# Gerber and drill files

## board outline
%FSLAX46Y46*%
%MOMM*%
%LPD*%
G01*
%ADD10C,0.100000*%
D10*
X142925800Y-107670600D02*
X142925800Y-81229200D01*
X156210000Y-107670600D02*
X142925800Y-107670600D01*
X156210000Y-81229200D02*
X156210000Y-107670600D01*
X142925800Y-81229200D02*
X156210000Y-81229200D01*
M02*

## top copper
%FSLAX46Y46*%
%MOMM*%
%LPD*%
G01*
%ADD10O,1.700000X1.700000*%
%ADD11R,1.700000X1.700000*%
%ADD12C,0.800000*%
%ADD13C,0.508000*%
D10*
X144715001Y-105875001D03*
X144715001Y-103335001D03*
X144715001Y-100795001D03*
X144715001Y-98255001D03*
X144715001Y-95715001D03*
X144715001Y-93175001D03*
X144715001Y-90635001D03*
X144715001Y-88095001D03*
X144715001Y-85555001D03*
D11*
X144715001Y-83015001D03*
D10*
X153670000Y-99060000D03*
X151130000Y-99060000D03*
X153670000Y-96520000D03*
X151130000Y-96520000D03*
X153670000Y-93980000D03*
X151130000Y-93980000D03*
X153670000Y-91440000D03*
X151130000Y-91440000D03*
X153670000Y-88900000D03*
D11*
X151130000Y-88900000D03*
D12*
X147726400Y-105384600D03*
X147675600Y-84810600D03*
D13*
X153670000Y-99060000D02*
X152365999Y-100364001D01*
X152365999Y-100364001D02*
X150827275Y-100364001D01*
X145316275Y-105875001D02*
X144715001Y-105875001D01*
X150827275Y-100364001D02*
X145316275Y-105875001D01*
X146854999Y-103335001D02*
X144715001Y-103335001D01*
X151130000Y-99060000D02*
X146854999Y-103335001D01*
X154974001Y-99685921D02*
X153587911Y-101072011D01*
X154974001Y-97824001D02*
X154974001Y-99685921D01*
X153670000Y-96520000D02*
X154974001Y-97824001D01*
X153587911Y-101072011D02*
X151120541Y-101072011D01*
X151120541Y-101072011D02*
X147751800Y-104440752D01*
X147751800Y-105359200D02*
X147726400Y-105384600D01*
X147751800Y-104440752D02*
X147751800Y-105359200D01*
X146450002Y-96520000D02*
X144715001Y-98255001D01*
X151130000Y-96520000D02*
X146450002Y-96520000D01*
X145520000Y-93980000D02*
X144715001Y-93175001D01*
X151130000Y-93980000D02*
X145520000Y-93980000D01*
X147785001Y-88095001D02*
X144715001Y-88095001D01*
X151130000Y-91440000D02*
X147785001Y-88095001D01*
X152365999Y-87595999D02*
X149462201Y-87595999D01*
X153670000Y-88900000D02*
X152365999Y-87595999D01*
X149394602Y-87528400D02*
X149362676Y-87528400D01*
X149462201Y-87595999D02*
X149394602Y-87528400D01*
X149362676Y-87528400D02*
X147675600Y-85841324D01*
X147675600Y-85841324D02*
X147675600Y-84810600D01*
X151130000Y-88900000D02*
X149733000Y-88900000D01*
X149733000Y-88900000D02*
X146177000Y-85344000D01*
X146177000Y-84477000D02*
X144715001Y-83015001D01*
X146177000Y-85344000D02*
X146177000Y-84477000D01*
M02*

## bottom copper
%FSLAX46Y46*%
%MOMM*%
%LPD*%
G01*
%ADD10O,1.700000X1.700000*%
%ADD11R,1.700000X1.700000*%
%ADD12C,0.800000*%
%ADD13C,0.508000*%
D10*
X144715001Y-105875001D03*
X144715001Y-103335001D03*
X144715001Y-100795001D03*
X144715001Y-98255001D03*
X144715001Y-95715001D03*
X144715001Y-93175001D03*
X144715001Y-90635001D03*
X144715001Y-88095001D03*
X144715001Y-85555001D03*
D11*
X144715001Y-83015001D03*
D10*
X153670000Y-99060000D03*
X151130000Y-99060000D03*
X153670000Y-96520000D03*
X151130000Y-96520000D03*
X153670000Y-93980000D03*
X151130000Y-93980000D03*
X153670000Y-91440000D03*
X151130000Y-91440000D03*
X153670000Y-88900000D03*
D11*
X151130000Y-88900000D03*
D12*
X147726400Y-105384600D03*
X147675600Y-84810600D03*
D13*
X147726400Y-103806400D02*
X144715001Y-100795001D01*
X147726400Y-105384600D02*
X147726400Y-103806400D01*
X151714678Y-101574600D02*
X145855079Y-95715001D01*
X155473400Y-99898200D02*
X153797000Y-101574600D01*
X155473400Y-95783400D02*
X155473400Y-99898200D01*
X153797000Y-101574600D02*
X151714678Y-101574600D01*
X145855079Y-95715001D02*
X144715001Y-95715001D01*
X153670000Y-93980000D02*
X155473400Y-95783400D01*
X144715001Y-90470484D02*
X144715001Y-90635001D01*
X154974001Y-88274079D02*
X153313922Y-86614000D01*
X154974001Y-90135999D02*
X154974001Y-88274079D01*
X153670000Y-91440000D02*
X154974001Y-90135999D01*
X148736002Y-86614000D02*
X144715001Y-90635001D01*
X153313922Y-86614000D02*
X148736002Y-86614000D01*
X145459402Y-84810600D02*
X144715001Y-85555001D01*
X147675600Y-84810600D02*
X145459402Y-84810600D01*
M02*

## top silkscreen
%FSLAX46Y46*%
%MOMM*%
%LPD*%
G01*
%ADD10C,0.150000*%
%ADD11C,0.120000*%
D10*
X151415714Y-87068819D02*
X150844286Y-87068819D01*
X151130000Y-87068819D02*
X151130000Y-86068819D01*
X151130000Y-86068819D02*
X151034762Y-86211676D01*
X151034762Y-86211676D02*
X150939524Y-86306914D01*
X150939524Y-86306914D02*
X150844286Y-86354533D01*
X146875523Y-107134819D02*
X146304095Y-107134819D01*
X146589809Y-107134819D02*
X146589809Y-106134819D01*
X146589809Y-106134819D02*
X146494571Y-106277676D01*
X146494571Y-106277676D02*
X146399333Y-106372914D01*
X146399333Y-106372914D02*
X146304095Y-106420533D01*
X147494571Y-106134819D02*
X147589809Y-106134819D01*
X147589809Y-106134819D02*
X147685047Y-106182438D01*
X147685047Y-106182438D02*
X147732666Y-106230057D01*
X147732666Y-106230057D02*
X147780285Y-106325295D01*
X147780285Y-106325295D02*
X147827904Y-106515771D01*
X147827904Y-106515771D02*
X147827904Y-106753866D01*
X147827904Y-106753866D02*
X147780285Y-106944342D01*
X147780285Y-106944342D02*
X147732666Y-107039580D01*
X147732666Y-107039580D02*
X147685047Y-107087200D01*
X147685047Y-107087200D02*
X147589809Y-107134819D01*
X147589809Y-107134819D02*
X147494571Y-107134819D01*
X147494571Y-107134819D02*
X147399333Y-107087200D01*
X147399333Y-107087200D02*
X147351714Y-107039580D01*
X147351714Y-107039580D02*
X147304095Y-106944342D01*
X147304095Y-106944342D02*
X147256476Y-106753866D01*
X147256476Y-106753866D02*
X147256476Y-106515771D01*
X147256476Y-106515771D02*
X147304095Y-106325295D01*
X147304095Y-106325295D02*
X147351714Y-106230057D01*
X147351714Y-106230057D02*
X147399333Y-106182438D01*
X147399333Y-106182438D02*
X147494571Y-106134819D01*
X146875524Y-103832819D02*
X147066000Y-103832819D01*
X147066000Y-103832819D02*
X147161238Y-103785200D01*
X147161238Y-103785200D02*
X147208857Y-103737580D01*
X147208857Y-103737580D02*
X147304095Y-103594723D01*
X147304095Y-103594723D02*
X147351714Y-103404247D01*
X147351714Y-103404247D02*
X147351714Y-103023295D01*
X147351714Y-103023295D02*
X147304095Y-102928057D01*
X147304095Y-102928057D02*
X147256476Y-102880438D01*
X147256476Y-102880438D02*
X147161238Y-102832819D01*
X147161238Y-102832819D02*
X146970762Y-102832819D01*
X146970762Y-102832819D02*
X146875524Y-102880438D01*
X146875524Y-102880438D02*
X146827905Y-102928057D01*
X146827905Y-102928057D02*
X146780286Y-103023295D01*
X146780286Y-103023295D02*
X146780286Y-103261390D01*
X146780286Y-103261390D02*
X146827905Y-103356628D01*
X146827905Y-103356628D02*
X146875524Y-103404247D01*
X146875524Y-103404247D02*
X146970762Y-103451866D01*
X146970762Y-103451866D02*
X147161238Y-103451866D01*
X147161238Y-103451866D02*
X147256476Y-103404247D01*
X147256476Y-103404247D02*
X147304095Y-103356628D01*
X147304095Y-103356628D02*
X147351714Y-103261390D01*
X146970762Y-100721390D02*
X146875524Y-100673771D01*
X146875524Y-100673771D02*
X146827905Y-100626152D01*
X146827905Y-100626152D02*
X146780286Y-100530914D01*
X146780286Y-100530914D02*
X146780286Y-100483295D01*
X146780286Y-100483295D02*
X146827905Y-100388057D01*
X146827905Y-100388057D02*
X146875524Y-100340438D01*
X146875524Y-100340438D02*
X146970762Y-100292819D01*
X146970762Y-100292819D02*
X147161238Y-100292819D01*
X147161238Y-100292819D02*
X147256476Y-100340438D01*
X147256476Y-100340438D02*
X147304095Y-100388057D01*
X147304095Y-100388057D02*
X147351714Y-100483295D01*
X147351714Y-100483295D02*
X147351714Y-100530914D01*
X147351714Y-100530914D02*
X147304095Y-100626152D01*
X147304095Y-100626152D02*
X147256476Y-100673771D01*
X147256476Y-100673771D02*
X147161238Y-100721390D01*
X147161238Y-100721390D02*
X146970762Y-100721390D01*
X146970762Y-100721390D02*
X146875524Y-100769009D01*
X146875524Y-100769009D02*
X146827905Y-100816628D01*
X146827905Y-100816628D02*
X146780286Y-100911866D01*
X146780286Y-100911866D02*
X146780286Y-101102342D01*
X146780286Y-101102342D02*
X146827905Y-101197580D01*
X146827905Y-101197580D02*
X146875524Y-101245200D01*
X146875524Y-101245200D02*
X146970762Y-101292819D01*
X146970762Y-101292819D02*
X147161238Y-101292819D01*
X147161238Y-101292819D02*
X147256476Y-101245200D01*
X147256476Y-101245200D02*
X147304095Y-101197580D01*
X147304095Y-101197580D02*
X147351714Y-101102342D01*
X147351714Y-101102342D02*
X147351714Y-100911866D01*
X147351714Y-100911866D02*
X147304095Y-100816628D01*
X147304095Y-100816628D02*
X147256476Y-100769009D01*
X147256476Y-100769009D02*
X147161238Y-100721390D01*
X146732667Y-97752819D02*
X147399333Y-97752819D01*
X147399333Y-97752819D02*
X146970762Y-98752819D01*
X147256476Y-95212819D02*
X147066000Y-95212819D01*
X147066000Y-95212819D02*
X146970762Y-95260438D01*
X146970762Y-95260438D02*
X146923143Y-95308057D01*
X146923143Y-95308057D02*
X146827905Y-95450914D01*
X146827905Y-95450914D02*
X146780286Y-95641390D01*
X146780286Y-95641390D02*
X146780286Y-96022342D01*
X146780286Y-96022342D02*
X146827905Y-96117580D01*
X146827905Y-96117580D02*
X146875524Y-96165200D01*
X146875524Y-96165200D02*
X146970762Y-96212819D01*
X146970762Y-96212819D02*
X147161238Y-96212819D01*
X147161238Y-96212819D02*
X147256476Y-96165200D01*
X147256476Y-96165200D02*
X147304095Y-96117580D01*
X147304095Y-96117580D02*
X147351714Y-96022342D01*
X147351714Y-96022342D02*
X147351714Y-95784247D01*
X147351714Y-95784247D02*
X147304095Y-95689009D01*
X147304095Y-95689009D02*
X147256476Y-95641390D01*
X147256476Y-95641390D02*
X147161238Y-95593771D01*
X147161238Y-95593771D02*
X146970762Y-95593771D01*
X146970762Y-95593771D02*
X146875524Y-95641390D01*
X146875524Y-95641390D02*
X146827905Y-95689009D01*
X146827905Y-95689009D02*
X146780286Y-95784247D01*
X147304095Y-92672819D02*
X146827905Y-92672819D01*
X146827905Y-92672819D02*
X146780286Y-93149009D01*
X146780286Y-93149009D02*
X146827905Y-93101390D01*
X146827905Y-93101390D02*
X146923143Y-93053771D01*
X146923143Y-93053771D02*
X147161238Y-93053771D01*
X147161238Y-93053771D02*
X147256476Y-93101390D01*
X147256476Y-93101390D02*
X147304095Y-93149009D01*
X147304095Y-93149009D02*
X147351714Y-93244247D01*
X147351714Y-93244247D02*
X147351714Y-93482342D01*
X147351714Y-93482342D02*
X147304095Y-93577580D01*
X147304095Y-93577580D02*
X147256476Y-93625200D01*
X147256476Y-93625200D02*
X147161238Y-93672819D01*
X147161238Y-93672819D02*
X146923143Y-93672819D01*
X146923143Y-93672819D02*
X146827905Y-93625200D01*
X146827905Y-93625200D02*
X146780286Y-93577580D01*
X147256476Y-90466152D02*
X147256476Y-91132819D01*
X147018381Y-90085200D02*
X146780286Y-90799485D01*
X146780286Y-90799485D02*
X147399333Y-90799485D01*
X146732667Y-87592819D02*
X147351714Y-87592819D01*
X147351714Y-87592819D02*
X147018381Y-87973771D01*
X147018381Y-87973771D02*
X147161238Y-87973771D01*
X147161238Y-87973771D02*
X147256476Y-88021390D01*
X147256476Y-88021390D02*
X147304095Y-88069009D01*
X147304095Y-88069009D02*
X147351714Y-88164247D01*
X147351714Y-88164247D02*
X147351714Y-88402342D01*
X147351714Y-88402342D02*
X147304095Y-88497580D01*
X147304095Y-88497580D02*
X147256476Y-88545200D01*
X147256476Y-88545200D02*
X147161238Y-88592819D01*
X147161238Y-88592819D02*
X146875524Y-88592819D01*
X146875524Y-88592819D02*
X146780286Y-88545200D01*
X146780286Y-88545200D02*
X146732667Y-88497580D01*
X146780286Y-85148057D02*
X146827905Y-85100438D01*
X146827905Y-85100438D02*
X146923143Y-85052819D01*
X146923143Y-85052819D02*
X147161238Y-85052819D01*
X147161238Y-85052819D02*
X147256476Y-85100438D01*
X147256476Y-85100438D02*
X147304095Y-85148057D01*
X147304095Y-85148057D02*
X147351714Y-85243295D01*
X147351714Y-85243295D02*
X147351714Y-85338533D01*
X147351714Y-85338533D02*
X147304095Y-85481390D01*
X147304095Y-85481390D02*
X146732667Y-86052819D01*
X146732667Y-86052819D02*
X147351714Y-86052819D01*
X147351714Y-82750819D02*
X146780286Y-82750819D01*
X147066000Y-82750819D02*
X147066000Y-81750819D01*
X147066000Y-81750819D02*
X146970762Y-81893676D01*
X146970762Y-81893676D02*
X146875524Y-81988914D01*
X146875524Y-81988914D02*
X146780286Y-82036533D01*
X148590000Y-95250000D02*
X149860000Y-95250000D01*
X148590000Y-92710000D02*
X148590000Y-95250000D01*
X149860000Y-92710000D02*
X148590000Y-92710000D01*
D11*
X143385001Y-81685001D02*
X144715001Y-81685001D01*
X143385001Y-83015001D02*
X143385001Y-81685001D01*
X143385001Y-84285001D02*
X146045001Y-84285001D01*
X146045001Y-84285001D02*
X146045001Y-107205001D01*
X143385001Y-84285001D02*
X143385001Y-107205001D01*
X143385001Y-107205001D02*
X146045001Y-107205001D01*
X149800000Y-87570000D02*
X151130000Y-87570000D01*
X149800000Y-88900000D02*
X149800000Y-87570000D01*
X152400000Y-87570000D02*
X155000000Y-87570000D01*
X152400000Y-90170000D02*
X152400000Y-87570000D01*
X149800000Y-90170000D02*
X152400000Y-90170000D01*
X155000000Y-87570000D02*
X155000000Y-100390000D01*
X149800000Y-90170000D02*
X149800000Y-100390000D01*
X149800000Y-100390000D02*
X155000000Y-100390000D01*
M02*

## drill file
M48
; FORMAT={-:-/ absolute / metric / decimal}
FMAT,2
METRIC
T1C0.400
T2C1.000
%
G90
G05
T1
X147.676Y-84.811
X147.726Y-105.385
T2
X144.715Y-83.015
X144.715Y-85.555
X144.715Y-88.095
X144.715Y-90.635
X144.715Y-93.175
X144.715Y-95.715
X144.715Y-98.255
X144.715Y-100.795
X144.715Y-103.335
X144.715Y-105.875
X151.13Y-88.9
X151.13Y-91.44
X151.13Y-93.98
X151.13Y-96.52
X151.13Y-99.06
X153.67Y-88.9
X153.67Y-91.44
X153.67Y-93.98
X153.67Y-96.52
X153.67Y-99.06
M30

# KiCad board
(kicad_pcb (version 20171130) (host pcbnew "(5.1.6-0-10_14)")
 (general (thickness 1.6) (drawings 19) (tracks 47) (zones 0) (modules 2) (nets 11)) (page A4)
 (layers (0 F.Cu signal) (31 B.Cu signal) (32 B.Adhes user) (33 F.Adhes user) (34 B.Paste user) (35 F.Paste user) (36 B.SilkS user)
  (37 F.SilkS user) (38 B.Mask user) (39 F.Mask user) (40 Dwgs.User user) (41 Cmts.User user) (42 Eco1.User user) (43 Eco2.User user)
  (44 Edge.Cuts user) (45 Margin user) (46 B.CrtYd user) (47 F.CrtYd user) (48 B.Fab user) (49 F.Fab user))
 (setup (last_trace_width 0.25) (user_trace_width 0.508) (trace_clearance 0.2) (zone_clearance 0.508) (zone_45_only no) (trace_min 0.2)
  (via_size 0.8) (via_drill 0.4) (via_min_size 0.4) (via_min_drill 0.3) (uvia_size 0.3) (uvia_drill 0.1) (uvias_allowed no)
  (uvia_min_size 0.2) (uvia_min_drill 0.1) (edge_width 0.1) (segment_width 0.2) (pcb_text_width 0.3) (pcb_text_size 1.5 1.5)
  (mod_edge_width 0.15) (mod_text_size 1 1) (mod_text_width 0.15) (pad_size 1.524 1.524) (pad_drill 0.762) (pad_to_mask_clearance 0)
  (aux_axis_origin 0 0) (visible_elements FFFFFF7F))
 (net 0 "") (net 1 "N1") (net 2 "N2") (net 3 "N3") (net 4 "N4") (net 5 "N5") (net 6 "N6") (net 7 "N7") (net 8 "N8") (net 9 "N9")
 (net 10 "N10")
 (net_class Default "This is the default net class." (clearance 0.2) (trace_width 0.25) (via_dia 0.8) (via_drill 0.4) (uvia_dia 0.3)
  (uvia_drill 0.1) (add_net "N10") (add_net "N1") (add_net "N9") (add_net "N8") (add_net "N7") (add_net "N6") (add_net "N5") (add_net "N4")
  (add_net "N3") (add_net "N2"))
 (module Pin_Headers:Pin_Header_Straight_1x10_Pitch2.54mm (layer F.Cu) (at 144.715001 83.015001)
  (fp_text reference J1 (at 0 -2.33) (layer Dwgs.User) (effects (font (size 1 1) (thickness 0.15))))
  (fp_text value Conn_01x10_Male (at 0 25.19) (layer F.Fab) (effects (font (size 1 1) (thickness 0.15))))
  (fp_line (start -1.33 -1.33) (end 0 -1.33) (layer F.SilkS) (width 0.12))
  (fp_line (start -1.33 0) (end -1.33 -1.33) (layer F.SilkS) (width 0.12))
  (fp_line (start -1.33 1.27) (end 1.33 1.27) (layer F.SilkS) (width 0.12))
  (fp_line (start 1.33 1.27) (end 1.33 24.19) (layer F.SilkS) (width 0.12))
  (fp_line (start -1.33 1.27) (end -1.33 24.19) (layer F.SilkS) (width 0.12))
  (fp_line (start -1.33 24.19) (end 1.33 24.19) (layer F.SilkS) (width 0.12))
  (pad 10 thru_hole oval (at 0 22.86) (size 1.7 1.7) (drill 1) (layers *.Cu *.Mask) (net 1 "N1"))
  (pad 9 thru_hole oval (at 0 20.32) (size 1.7 1.7) (drill 1) (layers *.Cu *.Mask) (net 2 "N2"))
  (pad 8 thru_hole oval (at 0 17.78) (size 1.7 1.7) (drill 1) (layers *.Cu *.Mask) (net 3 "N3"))
  (pad 7 thru_hole oval (at 0 15.24) (size 1.7 1.7) (drill 1) (layers *.Cu *.Mask) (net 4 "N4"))
  (pad 6 thru_hole oval (at 0 12.7) (size 1.7 1.7) (drill 1) (layers *.Cu *.Mask) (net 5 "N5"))
  (pad 5 thru_hole oval (at 0 10.16) (size 1.7 1.7) (drill 1) (layers *.Cu *.Mask) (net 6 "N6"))
  (pad 4 thru_hole oval (at 0 7.62) (size 1.7 1.7) (drill 1) (layers *.Cu *.Mask) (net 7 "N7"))
  (pad 3 thru_hole oval (at 0 5.08) (size 1.7 1.7) (drill 1) (layers *.Cu *.Mask) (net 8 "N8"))
  (pad 2 thru_hole oval (at 0 2.54) (size 1.7 1.7) (drill 1) (layers *.Cu *.Mask) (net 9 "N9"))
  (pad 1 thru_hole rect (at 0 0) (size 1.7 1.7) (drill 1) (layers *.Cu *.Mask) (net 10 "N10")))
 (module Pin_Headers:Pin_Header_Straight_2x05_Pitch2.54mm (layer F.Cu) (at 151.13 88.9)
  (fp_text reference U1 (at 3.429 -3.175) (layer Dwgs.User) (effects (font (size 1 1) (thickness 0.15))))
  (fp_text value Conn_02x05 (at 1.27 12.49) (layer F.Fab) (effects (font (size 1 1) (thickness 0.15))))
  (fp_line (start -1.33 -1.33) (end 0 -1.33) (layer F.SilkS) (width 0.12))
  (fp_line (start -1.33 0) (end -1.33 -1.33) (layer F.SilkS) (width 0.12))
  (fp_line (start 1.27 -1.33) (end 3.87 -1.33) (layer F.SilkS) (width 0.12))
  (fp_line (start 1.27 1.27) (end 1.27 -1.33) (layer F.SilkS) (width 0.12))
  (fp_line (start -1.33 1.27) (end 1.27 1.27) (layer F.SilkS) (width 0.12))
  (fp_line (start 3.87 -1.33) (end 3.87 11.49) (layer F.SilkS) (width 0.12))
  (fp_line (start -1.33 1.27) (end -1.33 11.49) (layer F.SilkS) (width 0.12))
  (fp_line (start -1.33 11.49) (end 3.87 11.49) (layer F.SilkS) (width 0.12))
  (pad 10 thru_hole oval (at 2.54 10.16) (size 1.7 1.7) (drill 1) (layers *.Cu *.Mask) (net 1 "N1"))
  (pad 9 thru_hole oval (at 0 10.16) (size 1.7 1.7) (drill 1) (layers *.Cu *.Mask) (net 2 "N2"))
  (pad 8 thru_hole oval (at 2.54 7.62) (size 1.7 1.7) (drill 1) (layers *.Cu *.Mask) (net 3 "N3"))
  (pad 7 thru_hole oval (at 0 7.62) (size 1.7 1.7) (drill 1) (layers *.Cu *.Mask) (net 4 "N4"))
  (pad 6 thru_hole oval (at 2.54 5.08) (size 1.7 1.7) (drill 1) (layers *.Cu *.Mask) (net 5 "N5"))
  (pad 5 thru_hole oval (at 0 5.08) (size 1.7 1.7) (drill 1) (layers *.Cu *.Mask) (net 6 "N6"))
  (pad 4 thru_hole oval (at 2.54 2.54) (size 1.7 1.7) (drill 1) (layers *.Cu *.Mask) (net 7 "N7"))
  (pad 3 thru_hole oval (at 0 2.54) (size 1.7 1.7) (drill 1) (layers *.Cu *.Mask) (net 8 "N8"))
  (pad 2 thru_hole oval (at 2.54 0) (size 1.7 1.7) (drill 1) (layers *.Cu *.Mask) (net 9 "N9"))
  (pad 1 thru_hole rect (at 0 0) (size 1.7 1.7) (drill 1) (layers *.Cu *.Mask) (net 10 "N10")))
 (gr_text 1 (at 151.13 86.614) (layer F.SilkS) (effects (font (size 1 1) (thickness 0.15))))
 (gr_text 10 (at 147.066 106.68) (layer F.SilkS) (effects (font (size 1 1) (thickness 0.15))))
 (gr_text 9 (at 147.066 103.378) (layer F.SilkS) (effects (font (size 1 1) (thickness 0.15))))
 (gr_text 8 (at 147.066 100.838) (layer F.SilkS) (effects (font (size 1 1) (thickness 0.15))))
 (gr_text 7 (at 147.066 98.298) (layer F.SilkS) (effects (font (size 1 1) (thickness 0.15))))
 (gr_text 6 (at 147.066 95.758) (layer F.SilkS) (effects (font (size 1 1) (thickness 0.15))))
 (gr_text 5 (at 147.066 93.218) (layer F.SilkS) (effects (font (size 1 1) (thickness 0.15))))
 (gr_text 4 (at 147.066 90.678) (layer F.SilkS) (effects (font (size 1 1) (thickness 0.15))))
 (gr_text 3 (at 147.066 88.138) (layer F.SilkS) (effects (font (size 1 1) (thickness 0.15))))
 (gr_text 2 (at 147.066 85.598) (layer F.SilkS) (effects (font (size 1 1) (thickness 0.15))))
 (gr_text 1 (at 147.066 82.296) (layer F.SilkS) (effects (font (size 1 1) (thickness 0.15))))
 (gr_line (start 142.9258 107.6706) (end 142.9258 81.2292) (layer Edge.Cuts) (width 0.1))
 (gr_line (start 156.21 107.6706) (end 142.9258 107.6706) (layer Edge.Cuts) (width 0.1))
 (gr_line (start 156.21 81.2292) (end 156.21 107.6706) (layer Edge.Cuts) (width 0.1))
 (gr_line (start 142.9258 81.2292) (end 156.21 81.2292) (layer Edge.Cuts) (width 0.1))
 (gr_line (start 148.59 95.25) (end 149.86 95.25) (layer F.SilkS) (width 0.15))
 (gr_line (start 148.59 92.71) (end 148.59 95.25) (layer F.SilkS) (width 0.15))
 (gr_line (start 149.86 92.71) (end 148.59 92.71) (layer F.SilkS) (width 0.15))
 (segment (start 153.67 99.06) (end 152.365999 100.364001) (width 0.508) (layer F.Cu) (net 1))
 (segment (start 152.365999 100.364001) (end 150.827275 100.364001) (width 0.508) (layer F.Cu) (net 1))
 (segment (start 145.316275 105.875001) (end 144.715001 105.875001) (width 0.508) (layer F.Cu) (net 1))
 (segment (start 150.827275 100.364001) (end 145.316275 105.875001) (width 0.508) (layer F.Cu) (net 1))
 (segment (start 146.854999 103.335001) (end 144.715001 103.335001) (width 0.508) (layer F.Cu) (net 2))
 (segment (start 151.13 99.06) (end 146.854999 103.335001) (width 0.508) (layer F.Cu) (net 2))
 (segment (start 154.974001 99.685921) (end 153.587911 101.072011) (width 0.508) (layer F.Cu) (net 3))
 (segment (start 154.974001 97.824001) (end 154.974001 99.685921) (width 0.508) (layer F.Cu) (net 3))
 (segment (start 153.67 96.52) (end 154.974001 97.824001) (width 0.508) (layer F.Cu) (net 3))
 (segment (start 153.587911 101.072011) (end 151.120541 101.072011) (width 0.508) (layer F.Cu) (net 3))
 (segment (start 151.120541 101.072011) (end 147.7518 104.440752) (width 0.508) (layer F.Cu) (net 3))
 (via (at 147.7264 105.3846) (size 0.8) (drill 0.4) (layers F.Cu B.Cu) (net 3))
 (segment (start 147.7518 105.3592) (end 147.7264 105.3846) (width 0.508) (layer F.Cu) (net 3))
 (segment (start 147.7518 104.440752) (end 147.7518 105.3592) (width 0.508) (layer F.Cu) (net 3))
 (segment (start 147.7264 103.8064) (end 144.715001 100.795001) (width 0.508) (layer B.Cu) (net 3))
 (segment (start 147.7264 105.3846) (end 147.7264 103.8064) (width 0.508) (layer B.Cu) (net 3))
 (segment (start 146.450002 96.52) (end 144.715001 98.255001) (width 0.508) (layer F.Cu) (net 4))
 (segment (start 151.13 96.52) (end 146.450002 96.52) (width 0.508) (layer F.Cu) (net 4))
 (segment (start 151.714678 101.5746) (end 145.855079 95.715001) (width 0.508) (layer B.Cu) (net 5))
 (segment (start 155.4734 99.8982) (end 153.797 101.5746) (width 0.508) (layer B.Cu) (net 5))
 (segment (start 155.4734 95.7834) (end 155.4734 99.8982) (width 0.508) (layer B.Cu) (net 5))
 (segment (start 153.797 101.5746) (end 151.714678 101.5746) (width 0.508) (layer B.Cu) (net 5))
 (segment (start 145.855079 95.715001) (end 144.715001 95.715001) (width 0.508) (layer B.Cu) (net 5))
 (segment (start 153.67 93.98) (end 155.4734 95.7834) (width 0.508) (layer B.Cu) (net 5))
 (segment (start 145.52 93.98) (end 144.715001 93.175001) (width 0.508) (layer F.Cu) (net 6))
 (segment (start 151.13 93.98) (end 145.52 93.98) (width 0.508) (layer F.Cu) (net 6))
 (segment (start 144.715001 90.470484) (end 144.715001 90.635001) (width 0.508) (layer B.Cu) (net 7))
 (segment (start 154.974001 88.274079) (end 153.313922 86.614) (width 0.508) (layer B.Cu) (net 7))
 (segment (start 154.974001 90.135999) (end 154.974001 88.274079) (width 0.508) (layer B.Cu) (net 7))
 (segment (start 153.67 91.44) (end 154.974001 90.135999) (width 0.508) (layer B.Cu) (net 7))
 (segment (start 148.736002 86.614) (end 144.715001 90.635001) (width 0.508) (layer B.Cu) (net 7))
 (segment (start 153.313922 86.614) (end 148.736002 86.614) (width 0.508) (layer B.Cu) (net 7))
 (segment (start 147.785001 88.095001) (end 144.715001 88.095001) (width 0.508) (layer F.Cu) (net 8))
 (segment (start 151.13 91.44) (end 147.785001 88.095001) (width 0.508) (layer F.Cu) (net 8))
 (segment (start 152.365999 87.595999) (end 149.462201 87.595999) (width 0.508) (layer F.Cu) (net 9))
 (segment (start 153.67 88.9) (end 152.365999 87.595999) (width 0.508) (layer F.Cu) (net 9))
 (segment (start 149.394602 87.5284) (end 149.362676 87.5284) (width 0.508) (layer F.Cu) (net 9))
 (segment (start 149.462201 87.595999) (end 149.394602 87.5284) (width 0.508) (layer F.Cu) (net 9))
 (segment (start 149.362676 87.5284) (end 147.6756 85.841324) (width 0.508) (layer F.Cu) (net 9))
 (via (at 147.6756 84.8106) (size 0.8) (drill 0.4) (layers F.Cu B.Cu) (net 9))
 (segment (start 147.6756 85.841324) (end 147.6756 84.8106) (width 0.508) (layer F.Cu) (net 9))
 (segment (start 145.459402 84.8106) (end 144.715001 85.555001) (width 0.508) (layer B.Cu) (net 9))
 (segment (start 147.6756 84.8106) (end 145.459402 84.8106) (width 0.508) (layer B.Cu) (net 9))
 (segment (start 151.13 88.9) (end 149.733 88.9) (width 0.508) (layer F.Cu) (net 10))
 (segment (start 149.733 88.9) (end 146.177 85.344) (width 0.508) (layer F.Cu) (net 10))
 (segment (start 146.177 84.477) (end 144.715001 83.015001) (width 0.508) (layer F.Cu) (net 10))
 (segment (start 146.177 85.344) (end 146.177 84.477) (width 0.508) (layer F.Cu) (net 10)))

